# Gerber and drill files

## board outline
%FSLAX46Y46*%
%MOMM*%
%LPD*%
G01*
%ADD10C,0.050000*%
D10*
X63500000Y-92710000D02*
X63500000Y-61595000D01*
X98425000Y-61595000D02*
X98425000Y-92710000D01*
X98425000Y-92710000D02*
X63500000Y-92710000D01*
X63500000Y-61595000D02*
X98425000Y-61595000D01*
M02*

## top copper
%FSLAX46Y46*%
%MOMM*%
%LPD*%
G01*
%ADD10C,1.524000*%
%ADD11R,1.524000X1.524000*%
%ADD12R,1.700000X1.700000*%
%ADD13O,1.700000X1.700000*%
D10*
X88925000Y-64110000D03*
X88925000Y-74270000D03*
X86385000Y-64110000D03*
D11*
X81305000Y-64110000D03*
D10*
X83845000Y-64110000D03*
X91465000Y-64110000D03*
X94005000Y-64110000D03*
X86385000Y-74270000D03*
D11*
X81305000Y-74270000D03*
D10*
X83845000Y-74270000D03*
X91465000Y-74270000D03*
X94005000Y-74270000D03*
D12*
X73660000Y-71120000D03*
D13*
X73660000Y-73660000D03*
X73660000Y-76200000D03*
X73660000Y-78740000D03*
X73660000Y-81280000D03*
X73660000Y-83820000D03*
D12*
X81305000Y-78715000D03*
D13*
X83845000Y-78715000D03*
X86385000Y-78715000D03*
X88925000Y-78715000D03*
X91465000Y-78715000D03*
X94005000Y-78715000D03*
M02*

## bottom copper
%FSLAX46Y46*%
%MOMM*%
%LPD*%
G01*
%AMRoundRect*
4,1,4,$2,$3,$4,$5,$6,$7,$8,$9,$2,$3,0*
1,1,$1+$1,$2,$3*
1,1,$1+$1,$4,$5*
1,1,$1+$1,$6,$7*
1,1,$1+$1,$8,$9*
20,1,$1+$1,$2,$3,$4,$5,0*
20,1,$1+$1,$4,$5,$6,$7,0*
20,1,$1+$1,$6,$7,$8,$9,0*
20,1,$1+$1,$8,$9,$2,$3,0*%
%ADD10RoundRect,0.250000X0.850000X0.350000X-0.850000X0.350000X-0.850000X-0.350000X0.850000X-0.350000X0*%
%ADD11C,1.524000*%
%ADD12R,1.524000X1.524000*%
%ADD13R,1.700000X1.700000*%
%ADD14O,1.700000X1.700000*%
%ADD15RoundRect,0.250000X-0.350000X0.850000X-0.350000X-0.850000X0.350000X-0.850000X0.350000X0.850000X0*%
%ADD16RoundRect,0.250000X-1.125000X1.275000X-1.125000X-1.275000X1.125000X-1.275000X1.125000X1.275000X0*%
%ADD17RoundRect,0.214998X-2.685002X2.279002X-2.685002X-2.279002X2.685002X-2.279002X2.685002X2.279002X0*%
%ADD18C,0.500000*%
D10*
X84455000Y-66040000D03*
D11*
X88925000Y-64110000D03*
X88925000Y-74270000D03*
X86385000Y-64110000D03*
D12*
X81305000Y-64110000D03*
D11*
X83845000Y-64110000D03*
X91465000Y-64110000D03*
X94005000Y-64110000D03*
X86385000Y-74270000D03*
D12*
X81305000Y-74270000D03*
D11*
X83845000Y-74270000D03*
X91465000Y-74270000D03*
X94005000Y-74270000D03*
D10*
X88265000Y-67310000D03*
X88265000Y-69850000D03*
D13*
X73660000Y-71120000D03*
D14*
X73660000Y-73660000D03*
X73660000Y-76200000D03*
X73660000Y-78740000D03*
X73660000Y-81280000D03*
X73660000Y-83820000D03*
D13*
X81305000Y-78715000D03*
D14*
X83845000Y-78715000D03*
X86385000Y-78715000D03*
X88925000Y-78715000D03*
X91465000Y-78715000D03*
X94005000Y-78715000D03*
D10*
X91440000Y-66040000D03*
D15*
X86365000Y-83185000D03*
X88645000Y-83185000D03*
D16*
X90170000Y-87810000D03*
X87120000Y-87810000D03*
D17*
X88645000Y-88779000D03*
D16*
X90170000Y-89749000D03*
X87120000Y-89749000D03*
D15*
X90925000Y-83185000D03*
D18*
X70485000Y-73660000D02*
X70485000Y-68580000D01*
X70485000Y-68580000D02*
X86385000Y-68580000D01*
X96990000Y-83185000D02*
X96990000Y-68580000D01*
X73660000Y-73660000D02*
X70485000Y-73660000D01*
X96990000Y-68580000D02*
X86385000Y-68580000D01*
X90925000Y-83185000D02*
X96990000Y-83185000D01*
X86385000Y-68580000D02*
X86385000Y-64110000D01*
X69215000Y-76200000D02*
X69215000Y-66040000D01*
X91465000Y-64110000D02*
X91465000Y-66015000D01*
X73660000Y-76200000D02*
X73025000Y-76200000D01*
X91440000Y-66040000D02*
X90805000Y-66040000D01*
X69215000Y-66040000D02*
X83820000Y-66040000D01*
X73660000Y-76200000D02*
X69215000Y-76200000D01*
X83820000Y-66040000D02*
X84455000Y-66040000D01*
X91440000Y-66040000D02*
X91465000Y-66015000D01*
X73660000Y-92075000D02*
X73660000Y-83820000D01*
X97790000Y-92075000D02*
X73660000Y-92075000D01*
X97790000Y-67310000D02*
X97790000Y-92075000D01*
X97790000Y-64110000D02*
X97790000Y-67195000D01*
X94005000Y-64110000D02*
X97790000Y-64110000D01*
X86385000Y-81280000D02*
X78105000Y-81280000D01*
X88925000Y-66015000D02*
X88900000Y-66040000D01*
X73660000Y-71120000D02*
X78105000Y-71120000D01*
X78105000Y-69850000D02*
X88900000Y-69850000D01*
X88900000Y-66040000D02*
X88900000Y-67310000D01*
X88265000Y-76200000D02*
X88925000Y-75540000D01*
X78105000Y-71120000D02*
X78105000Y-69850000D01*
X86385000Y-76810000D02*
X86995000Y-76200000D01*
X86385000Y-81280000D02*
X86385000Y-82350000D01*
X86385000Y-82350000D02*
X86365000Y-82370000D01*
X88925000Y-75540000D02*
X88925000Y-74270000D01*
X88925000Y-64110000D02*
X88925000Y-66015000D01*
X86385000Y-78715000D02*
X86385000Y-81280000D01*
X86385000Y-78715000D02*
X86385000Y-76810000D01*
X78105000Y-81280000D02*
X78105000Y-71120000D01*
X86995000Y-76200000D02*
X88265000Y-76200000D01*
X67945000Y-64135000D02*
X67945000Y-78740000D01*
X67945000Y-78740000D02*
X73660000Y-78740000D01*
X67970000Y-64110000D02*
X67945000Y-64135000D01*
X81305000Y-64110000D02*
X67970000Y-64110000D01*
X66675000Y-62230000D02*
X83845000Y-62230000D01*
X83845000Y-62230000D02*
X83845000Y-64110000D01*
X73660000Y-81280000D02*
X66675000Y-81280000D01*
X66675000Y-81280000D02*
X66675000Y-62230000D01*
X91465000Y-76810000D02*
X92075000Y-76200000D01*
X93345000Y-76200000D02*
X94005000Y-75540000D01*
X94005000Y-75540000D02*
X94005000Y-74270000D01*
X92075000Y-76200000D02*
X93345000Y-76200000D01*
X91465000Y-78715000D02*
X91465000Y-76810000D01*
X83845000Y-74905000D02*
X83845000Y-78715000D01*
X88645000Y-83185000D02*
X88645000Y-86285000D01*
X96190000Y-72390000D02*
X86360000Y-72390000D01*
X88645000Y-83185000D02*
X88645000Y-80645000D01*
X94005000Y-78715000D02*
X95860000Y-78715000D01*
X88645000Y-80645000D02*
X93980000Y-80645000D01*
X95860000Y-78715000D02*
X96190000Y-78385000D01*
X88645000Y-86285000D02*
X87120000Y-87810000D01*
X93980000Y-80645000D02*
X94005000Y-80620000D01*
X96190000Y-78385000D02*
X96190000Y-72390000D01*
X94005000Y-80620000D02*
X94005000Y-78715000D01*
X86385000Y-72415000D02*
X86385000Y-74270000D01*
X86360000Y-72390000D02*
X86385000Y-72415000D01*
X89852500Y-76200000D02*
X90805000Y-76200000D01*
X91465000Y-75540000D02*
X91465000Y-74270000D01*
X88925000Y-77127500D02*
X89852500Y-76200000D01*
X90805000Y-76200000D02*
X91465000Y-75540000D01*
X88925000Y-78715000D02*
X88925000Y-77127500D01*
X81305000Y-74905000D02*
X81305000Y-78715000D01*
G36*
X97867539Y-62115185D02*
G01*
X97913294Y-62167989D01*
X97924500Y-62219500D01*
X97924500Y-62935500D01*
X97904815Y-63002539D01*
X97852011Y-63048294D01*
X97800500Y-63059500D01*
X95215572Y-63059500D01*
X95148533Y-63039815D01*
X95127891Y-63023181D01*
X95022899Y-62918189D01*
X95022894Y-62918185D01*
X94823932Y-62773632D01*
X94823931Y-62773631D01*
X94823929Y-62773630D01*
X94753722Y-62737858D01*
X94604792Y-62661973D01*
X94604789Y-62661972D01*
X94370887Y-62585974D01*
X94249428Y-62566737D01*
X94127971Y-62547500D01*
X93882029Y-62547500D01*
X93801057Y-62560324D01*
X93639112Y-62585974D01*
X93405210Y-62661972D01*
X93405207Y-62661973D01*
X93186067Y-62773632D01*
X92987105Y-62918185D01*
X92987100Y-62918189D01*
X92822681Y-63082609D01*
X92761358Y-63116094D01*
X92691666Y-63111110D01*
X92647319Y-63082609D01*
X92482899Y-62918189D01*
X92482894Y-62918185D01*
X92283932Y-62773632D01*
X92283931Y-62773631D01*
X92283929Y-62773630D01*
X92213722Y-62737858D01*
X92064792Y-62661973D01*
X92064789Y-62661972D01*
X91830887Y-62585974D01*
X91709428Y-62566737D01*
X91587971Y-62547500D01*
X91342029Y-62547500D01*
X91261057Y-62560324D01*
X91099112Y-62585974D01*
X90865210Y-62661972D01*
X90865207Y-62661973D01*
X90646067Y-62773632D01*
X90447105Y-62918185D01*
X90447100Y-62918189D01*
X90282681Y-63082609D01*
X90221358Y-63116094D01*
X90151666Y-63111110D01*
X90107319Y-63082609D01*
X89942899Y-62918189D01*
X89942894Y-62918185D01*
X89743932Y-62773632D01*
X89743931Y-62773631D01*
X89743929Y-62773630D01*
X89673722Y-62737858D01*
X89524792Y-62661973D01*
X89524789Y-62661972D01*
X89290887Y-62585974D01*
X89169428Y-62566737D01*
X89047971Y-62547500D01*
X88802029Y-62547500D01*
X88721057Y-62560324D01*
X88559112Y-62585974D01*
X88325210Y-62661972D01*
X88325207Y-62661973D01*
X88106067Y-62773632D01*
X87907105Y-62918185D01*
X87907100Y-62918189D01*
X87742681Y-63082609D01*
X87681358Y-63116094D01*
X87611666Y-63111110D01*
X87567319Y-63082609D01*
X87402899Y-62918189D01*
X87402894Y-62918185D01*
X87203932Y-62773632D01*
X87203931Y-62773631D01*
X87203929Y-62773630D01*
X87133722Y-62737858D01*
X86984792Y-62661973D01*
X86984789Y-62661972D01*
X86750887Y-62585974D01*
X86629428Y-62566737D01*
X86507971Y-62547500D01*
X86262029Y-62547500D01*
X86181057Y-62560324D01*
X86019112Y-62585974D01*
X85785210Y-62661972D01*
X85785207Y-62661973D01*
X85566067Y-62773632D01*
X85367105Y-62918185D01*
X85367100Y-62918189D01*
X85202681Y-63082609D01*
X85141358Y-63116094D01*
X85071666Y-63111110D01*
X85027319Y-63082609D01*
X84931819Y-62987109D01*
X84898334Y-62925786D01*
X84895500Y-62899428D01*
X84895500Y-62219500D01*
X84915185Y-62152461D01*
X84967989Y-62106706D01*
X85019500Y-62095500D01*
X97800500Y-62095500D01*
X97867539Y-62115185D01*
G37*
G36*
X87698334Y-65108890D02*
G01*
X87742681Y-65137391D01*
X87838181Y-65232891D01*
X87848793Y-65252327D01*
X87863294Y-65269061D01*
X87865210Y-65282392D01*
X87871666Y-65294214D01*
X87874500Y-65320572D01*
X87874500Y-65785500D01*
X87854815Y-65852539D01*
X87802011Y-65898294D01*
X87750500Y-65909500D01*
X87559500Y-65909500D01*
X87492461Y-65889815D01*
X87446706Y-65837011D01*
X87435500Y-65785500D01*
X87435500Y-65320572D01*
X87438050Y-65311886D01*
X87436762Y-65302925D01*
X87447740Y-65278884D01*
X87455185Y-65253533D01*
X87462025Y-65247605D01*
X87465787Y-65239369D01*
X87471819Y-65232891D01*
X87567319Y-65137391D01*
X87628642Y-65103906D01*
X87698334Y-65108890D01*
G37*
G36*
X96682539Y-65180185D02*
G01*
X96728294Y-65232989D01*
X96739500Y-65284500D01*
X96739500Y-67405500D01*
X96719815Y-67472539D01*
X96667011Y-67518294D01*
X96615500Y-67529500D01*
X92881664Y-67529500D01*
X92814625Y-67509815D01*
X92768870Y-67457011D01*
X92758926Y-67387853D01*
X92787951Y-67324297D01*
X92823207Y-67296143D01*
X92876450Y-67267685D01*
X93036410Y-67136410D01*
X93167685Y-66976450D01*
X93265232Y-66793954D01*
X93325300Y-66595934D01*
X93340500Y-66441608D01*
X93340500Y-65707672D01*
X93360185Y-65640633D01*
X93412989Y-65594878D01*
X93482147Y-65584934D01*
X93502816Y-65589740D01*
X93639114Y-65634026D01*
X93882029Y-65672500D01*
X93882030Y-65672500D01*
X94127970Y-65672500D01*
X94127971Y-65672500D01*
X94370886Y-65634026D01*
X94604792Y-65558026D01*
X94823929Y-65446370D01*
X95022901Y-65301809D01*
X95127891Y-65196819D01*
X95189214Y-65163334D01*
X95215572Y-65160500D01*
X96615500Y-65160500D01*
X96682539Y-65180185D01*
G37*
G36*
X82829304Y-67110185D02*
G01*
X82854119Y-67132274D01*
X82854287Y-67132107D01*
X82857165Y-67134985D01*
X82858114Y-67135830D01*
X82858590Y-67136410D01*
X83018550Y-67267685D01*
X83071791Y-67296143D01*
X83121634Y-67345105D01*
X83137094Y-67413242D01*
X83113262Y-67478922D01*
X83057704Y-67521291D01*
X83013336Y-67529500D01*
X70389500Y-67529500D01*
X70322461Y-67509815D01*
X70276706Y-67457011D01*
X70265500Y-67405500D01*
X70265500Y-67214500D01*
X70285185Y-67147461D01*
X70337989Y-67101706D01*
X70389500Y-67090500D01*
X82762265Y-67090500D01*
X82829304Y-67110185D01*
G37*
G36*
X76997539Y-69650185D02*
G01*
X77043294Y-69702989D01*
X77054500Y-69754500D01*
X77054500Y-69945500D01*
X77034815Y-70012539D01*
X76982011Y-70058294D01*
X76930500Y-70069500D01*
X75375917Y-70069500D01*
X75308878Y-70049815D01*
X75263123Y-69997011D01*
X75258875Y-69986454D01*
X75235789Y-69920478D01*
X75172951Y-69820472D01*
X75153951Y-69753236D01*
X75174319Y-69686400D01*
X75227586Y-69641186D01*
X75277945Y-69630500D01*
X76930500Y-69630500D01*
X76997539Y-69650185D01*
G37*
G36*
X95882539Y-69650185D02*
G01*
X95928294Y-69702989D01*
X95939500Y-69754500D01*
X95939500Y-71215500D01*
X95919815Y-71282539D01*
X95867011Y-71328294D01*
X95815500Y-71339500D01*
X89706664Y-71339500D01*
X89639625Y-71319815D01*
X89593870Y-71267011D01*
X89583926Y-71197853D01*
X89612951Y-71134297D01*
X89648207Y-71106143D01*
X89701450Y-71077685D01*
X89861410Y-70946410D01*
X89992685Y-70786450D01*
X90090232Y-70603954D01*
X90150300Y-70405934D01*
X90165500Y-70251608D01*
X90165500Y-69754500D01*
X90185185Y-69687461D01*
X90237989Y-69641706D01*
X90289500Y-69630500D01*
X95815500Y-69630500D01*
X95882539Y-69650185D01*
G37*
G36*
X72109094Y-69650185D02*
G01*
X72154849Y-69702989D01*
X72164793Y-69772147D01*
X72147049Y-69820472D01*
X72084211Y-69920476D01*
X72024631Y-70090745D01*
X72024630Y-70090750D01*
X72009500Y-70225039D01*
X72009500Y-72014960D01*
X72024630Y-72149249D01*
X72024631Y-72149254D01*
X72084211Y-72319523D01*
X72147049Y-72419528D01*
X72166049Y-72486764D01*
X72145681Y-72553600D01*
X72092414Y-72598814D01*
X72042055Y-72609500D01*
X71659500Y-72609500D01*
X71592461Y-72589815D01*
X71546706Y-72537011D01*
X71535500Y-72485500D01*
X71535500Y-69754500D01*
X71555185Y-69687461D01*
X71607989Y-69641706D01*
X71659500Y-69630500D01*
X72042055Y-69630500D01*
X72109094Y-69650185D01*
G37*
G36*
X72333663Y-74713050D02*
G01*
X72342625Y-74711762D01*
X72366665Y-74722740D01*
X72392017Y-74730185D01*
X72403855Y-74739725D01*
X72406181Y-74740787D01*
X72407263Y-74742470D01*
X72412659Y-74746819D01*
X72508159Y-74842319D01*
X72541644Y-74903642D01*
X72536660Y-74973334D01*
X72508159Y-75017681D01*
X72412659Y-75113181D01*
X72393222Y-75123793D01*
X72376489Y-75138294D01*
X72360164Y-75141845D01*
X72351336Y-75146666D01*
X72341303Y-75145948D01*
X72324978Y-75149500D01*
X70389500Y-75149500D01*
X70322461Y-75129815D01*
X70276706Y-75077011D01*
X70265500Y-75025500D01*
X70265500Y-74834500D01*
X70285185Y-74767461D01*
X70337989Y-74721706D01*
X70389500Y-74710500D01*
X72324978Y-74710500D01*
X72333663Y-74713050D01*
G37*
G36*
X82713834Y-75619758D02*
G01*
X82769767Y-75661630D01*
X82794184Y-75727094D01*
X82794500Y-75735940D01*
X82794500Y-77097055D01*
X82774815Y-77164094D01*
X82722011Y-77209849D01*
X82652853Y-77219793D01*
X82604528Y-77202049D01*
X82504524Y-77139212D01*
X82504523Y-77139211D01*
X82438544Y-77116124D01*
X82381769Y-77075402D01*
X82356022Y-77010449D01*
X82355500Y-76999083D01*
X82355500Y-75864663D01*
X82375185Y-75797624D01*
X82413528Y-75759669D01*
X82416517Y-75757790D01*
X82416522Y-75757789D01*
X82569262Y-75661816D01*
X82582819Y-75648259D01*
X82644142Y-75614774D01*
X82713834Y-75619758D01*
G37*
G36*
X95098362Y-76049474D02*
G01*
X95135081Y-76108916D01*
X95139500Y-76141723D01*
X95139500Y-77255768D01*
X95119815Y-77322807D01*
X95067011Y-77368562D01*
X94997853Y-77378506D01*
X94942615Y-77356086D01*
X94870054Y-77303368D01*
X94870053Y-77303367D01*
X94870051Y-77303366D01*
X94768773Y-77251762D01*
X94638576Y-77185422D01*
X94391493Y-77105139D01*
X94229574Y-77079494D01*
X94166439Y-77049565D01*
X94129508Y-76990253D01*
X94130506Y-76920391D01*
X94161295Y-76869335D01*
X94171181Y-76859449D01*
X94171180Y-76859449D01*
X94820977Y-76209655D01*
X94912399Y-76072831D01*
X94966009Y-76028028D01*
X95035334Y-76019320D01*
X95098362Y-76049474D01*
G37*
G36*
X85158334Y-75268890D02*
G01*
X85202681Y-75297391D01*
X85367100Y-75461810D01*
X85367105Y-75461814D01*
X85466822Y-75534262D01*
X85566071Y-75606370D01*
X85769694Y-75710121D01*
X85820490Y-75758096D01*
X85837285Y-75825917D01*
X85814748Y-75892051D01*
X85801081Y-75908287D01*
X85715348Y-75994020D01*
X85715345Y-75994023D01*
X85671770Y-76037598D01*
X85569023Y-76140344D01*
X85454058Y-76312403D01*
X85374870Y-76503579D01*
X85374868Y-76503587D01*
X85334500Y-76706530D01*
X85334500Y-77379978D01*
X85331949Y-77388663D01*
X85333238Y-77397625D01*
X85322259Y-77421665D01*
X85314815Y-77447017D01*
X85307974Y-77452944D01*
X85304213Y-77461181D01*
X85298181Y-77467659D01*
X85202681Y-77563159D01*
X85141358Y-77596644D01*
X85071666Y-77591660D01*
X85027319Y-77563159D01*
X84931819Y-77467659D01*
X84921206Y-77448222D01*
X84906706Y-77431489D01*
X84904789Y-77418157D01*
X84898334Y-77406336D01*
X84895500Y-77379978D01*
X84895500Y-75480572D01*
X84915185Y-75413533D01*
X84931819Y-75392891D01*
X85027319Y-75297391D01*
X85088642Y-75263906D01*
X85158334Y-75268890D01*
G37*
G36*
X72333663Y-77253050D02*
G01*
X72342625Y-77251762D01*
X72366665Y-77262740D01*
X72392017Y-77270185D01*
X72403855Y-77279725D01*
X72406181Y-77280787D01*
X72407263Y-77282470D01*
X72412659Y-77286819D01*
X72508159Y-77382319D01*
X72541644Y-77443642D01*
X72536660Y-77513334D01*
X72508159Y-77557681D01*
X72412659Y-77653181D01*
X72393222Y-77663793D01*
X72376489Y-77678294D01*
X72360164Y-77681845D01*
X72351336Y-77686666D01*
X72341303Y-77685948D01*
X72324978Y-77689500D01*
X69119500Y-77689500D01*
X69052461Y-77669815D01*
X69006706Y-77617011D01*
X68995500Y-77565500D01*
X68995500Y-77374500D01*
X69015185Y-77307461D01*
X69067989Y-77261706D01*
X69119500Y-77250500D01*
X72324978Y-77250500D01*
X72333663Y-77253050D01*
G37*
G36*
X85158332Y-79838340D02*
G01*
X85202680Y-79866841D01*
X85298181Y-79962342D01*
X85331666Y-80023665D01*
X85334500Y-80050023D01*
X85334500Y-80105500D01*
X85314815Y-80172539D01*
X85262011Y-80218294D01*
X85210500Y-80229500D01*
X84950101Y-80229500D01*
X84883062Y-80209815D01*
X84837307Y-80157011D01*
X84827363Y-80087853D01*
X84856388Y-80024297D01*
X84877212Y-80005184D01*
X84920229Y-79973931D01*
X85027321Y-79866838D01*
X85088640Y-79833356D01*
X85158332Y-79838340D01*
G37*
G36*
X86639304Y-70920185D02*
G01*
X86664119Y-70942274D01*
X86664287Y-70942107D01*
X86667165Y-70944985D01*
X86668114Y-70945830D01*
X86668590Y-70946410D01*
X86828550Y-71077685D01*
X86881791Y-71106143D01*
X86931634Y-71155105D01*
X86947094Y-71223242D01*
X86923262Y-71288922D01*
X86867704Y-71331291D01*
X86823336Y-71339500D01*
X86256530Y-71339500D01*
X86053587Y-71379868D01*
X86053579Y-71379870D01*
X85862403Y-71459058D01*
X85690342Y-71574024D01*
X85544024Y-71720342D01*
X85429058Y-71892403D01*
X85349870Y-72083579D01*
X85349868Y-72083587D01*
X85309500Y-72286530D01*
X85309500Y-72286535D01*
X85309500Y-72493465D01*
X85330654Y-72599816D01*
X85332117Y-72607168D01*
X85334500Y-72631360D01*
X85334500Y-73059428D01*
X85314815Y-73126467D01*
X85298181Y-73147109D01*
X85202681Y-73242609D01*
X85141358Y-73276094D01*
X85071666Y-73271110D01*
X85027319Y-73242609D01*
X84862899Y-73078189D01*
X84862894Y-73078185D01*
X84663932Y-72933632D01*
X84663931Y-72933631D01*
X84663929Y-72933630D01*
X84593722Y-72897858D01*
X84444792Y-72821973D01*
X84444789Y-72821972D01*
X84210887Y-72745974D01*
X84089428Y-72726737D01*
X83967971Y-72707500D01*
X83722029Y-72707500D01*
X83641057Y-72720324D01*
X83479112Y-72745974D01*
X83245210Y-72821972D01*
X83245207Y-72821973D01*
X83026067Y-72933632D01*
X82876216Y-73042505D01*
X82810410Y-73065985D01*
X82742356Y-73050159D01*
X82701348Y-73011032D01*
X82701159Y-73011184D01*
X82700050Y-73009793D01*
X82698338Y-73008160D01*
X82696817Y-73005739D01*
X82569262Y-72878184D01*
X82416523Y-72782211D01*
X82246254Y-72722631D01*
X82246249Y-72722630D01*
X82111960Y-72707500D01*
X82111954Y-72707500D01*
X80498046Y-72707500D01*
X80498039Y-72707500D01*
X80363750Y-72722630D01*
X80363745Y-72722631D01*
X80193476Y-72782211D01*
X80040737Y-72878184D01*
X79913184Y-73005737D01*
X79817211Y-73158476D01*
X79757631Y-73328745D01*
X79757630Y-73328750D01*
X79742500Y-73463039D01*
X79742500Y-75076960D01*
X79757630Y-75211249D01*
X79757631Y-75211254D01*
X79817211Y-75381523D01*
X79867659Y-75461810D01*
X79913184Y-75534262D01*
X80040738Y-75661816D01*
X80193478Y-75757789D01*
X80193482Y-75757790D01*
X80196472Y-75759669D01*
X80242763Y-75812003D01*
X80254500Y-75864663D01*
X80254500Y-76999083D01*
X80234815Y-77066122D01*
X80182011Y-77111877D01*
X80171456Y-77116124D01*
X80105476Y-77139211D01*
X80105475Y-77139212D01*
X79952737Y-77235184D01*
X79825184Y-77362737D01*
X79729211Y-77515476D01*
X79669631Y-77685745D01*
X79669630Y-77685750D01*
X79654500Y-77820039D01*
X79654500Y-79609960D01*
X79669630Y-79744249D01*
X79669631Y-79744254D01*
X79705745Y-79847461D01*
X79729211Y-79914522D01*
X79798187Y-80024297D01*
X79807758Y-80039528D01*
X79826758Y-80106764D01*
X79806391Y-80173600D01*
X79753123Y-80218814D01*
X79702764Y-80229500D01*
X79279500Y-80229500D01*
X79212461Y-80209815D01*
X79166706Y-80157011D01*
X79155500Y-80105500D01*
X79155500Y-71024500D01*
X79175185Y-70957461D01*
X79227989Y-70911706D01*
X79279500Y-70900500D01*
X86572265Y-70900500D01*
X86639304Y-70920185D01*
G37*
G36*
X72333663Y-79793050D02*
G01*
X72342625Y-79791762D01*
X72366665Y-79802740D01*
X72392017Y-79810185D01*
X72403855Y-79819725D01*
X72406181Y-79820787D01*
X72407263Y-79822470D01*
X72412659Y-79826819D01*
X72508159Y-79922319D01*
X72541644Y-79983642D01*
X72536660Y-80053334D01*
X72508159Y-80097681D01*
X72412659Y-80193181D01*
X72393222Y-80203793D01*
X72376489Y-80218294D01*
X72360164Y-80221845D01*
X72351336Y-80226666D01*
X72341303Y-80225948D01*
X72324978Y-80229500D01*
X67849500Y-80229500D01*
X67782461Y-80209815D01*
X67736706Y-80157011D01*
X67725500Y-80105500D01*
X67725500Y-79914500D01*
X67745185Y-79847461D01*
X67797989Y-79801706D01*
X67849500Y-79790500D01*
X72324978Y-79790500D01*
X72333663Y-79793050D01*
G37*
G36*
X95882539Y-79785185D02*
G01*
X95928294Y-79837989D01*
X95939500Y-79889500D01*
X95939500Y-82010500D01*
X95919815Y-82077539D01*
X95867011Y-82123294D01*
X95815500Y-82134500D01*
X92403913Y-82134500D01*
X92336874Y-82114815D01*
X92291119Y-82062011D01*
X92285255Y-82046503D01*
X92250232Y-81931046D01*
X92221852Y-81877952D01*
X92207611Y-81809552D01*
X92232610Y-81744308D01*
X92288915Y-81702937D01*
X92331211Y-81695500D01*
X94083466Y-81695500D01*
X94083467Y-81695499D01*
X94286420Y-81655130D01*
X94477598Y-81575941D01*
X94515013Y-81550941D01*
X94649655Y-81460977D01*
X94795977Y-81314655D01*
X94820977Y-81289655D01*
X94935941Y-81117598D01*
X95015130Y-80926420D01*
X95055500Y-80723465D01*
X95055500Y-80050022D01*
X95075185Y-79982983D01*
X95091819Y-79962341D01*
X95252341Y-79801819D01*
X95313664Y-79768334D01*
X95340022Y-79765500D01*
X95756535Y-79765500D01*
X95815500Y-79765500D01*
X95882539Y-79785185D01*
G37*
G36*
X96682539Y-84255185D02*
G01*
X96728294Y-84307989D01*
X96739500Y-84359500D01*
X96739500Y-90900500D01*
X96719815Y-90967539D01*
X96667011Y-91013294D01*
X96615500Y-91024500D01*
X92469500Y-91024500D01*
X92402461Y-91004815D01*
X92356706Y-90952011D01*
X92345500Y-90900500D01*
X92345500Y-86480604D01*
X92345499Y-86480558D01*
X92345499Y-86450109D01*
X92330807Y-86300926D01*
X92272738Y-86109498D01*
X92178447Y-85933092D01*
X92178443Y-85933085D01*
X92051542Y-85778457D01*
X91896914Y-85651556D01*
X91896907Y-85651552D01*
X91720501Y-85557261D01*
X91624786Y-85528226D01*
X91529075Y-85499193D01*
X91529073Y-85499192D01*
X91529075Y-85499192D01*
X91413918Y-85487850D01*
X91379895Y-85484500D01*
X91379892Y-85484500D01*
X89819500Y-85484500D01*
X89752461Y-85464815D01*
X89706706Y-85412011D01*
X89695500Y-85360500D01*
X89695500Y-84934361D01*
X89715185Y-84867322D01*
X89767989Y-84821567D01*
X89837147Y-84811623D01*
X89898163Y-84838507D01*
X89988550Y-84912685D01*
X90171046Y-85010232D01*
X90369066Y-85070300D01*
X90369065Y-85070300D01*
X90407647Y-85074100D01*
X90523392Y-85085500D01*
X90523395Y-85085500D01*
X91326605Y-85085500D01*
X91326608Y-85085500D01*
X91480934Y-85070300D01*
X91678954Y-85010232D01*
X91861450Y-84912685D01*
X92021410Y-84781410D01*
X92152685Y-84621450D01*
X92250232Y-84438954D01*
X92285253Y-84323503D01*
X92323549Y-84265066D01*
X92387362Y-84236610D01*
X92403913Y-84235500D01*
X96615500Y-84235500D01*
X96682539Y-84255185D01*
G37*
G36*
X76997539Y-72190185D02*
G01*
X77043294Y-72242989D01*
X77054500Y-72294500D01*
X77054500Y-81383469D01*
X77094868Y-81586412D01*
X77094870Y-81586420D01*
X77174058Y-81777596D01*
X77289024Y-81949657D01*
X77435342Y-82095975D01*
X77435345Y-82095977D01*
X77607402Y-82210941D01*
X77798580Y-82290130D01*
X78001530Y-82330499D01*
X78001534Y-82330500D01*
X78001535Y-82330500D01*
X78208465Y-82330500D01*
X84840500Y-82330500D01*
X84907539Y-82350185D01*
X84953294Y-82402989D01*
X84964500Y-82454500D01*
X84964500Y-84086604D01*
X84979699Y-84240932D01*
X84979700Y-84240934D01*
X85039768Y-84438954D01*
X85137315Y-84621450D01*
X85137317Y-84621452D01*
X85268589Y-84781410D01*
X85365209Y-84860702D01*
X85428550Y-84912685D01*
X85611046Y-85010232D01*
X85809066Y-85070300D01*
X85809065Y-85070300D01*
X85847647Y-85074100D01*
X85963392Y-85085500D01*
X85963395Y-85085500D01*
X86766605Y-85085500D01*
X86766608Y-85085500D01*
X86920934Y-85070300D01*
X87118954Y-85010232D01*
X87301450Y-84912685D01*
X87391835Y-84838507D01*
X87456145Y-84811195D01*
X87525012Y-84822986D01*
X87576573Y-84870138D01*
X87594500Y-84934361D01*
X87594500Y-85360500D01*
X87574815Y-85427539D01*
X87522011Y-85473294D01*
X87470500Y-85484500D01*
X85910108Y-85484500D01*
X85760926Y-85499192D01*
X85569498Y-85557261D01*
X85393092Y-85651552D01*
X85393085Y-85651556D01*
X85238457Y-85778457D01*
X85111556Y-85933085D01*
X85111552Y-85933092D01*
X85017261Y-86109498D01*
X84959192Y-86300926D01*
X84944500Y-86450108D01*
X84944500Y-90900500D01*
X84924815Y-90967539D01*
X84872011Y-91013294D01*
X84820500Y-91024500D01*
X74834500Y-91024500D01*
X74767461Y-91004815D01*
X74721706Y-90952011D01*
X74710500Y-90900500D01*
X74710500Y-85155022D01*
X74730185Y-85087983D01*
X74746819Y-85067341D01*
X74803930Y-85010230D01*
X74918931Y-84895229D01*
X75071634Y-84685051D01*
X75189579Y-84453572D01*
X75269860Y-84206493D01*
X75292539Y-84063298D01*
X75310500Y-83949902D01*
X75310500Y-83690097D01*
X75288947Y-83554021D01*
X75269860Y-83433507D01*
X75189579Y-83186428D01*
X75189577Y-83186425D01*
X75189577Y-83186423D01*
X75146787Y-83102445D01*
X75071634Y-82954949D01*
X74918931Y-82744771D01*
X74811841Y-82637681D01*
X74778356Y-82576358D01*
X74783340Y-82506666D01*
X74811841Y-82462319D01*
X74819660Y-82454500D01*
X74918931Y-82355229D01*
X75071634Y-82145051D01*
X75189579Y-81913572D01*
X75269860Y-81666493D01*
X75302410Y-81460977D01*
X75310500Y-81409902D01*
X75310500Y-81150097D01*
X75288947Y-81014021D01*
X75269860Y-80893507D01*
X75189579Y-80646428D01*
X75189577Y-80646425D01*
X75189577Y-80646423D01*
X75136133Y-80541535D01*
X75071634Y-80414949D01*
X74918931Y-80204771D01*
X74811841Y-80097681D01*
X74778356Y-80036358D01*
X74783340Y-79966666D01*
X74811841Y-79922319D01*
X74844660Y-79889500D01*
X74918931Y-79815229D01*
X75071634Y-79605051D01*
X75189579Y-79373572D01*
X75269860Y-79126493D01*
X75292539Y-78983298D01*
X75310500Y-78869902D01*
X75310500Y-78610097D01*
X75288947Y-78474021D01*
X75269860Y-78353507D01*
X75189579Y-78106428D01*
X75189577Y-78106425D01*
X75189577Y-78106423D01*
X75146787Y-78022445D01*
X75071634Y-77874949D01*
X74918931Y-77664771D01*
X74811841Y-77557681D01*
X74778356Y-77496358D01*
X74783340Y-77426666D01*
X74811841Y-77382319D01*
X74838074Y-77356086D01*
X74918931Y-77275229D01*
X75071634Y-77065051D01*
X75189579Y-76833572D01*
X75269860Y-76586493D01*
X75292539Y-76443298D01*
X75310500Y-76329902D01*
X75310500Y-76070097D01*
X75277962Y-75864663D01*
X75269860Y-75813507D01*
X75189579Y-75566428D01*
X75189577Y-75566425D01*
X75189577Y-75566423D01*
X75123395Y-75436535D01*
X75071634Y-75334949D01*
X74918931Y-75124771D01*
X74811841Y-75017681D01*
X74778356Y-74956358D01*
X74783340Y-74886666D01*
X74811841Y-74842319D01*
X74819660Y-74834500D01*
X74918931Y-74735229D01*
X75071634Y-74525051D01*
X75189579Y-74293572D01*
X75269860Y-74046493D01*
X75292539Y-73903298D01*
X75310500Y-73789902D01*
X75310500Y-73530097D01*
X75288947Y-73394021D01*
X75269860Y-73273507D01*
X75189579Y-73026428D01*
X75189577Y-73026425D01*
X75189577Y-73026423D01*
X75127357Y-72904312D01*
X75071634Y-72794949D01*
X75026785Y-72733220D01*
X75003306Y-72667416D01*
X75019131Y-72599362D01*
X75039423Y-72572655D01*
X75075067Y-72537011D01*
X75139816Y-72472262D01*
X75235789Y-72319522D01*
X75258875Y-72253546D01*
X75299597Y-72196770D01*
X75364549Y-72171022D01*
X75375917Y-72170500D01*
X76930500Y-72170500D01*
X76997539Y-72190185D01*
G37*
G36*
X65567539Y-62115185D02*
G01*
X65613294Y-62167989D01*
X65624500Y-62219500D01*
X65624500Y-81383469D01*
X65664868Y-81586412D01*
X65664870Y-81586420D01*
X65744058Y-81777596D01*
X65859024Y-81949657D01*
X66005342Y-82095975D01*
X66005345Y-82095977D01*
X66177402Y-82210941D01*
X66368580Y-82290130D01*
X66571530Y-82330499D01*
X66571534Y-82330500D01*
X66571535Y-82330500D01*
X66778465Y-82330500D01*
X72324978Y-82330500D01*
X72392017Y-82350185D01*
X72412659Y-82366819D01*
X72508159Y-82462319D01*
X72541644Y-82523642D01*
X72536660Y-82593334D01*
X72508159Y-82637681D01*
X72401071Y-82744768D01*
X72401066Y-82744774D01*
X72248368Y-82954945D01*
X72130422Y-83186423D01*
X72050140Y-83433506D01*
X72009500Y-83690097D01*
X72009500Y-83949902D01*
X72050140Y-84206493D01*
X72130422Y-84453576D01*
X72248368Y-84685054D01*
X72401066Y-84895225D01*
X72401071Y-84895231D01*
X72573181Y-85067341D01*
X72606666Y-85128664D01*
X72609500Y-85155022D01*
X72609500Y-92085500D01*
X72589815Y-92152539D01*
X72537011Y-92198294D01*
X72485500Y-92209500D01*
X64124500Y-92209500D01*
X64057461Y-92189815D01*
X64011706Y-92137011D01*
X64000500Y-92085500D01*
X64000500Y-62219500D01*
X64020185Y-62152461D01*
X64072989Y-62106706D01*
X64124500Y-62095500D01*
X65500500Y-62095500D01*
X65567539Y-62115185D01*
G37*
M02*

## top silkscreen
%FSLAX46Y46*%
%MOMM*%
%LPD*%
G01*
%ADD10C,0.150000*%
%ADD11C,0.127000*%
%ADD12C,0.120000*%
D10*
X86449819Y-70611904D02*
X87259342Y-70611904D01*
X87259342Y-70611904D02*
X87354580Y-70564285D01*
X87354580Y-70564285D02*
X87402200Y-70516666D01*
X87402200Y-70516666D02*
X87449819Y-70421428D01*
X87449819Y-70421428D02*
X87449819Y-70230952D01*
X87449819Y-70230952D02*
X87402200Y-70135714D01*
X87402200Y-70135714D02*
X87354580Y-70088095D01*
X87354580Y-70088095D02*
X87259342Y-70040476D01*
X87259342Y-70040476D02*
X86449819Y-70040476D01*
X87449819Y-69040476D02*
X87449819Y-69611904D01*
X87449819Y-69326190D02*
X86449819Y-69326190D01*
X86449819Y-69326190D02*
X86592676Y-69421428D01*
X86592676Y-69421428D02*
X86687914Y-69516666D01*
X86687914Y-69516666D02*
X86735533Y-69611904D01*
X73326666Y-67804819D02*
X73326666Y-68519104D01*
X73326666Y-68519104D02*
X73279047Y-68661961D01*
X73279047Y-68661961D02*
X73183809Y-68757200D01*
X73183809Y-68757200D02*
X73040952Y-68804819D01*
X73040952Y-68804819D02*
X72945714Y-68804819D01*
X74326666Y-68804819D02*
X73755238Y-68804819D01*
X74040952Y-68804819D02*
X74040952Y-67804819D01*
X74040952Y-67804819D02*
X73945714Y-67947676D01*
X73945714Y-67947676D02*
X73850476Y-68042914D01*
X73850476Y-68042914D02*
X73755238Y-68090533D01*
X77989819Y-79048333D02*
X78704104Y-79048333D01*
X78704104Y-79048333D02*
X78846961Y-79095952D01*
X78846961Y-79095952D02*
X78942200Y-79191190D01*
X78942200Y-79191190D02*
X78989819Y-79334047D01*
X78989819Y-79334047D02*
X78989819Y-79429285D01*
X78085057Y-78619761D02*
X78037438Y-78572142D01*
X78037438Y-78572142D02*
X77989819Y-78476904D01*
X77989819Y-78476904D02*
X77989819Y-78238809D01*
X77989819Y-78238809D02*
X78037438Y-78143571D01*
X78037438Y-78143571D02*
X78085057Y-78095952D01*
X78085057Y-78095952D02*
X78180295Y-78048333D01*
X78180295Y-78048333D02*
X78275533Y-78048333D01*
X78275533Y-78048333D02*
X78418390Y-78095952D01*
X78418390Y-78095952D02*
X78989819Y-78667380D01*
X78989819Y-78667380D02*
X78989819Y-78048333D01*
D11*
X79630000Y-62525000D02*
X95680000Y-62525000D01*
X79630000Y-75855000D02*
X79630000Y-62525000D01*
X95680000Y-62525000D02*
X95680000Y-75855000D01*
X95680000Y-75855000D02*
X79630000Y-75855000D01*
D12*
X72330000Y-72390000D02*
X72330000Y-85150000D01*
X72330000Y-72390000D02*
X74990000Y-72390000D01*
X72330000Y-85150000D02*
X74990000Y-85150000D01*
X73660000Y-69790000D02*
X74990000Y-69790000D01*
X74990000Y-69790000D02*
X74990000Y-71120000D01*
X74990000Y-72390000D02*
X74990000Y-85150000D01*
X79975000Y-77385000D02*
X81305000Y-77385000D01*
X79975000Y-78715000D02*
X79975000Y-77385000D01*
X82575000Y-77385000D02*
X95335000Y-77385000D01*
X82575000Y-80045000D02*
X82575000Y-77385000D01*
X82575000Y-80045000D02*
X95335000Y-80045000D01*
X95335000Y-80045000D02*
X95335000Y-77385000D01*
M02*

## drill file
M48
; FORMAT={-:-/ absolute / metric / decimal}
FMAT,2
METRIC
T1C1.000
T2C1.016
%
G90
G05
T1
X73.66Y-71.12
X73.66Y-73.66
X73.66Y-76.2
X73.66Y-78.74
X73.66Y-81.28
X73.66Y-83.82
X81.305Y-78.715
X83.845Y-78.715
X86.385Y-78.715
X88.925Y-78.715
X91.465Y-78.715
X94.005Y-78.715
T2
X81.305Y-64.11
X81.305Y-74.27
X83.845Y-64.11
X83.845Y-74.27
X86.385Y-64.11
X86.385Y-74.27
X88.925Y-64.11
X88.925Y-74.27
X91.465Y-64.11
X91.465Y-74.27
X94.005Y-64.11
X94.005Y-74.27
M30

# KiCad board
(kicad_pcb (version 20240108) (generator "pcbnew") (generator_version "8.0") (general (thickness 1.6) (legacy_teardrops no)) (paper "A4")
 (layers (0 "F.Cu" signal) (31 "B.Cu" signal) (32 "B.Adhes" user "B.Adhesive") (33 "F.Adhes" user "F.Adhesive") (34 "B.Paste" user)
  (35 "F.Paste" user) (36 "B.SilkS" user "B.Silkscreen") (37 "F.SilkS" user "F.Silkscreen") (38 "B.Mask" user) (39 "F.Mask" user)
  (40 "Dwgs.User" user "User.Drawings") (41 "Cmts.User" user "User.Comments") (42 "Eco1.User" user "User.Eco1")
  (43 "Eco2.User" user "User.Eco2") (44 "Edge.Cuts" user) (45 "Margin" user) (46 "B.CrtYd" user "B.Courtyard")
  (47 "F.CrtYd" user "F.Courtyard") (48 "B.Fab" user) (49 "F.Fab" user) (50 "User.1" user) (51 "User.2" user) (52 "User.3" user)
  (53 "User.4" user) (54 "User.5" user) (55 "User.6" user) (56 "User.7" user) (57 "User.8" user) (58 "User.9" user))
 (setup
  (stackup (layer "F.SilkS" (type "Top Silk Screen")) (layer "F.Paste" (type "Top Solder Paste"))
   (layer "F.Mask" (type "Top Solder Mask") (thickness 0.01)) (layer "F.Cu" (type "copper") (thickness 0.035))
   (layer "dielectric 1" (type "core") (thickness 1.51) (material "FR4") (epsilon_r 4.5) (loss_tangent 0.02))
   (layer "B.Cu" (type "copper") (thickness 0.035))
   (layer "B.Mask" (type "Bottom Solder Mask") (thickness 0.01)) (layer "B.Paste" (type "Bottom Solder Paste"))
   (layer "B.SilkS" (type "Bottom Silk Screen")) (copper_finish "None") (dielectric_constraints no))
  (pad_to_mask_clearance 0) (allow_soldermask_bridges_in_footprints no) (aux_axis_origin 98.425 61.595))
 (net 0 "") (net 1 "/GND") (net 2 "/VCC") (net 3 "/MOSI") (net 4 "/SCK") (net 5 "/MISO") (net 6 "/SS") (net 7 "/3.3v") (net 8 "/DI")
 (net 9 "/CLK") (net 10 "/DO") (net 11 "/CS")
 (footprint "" (layer "F.Cu") (at 84.455 66.04 -90)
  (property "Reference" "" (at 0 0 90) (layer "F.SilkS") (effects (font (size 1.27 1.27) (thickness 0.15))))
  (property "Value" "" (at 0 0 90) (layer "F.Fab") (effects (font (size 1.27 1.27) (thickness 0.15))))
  (pad "1" smd roundrect (at 0 0 180) (size 2.2 1.2) (layers "B.Cu" "B.Paste" "B.Mask") (roundrect_rratio 0.208333)))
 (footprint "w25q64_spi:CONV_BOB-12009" (layer "F.Cu") (at 87.655 69.19 90)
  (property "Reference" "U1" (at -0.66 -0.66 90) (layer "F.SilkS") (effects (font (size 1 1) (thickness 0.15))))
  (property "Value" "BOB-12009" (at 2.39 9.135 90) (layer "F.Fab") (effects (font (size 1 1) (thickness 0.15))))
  (fp_line (start 6.665 -8.025) (end 6.665 8.025) (stroke (width 0.127) (type solid)) (layer "F.SilkS"))
  (fp_line (start -6.665 -8.025) (end 6.665 -8.025) (stroke (width 0.127) (type solid)) (layer "F.SilkS"))
  (fp_line (start 6.665 8.025) (end -6.665 8.025) (stroke (width 0.127) (type solid)) (layer "F.SilkS"))
  (fp_line (start -6.665 8.025) (end -6.665 -8.025) (stroke (width 0.127) (type solid)) (layer "F.SilkS"))
  (pad "GND_1" thru_hole circle (at 5.08 1.27 90) (size 1.524 1.524) (drill 1.016) (layers "*.Cu" "*.Mask") (remove_unused_layers no)
   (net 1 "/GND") (solder_mask_margin 0.102))
  (pad "GND_2" thru_hole circle (at -5.08 1.27 90) (size 1.524 1.524) (drill 1.016) (layers "*.Cu" "*.Mask") (remove_unused_layers no)
   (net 1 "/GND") (solder_mask_margin 0.102))
  (pad "HV" thru_hole circle (at 5.08 -1.27 90) (size 1.524 1.524) (drill 1.016) (layers "*.Cu" "*.Mask") (remove_unused_layers no)
   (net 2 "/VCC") (solder_mask_margin 0.102))
  (pad "HV1" thru_hole rect (at 5.08 -6.35 90) (size 1.524 1.524) (drill 1.016) (layers "*.Cu" "*.Mask") (remove_unused_layers no)
   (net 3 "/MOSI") (solder_mask_margin 0.102))
  (pad "HV2" thru_hole circle (at 5.08 -3.81 90) (size 1.524 1.524) (drill 1.016) (layers "*.Cu" "*.Mask") (remove_unused_layers no)
   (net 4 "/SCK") (solder_mask_margin 0.102))
  (pad "HV3" thru_hole circle (at 5.08 3.81 90) (size 1.524 1.524) (drill 1.016) (layers "*.Cu" "*.Mask") (remove_unused_layers no)
   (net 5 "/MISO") (solder_mask_margin 0.102))
  (pad "HV4" thru_hole circle (at 5.08 6.35 90) (size 1.524 1.524) (drill 1.016) (layers "*.Cu" "*.Mask") (remove_unused_layers no)
   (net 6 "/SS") (solder_mask_margin 0.102))
  (pad "LV" thru_hole circle (at -5.08 -1.27 90) (size 1.524 1.524) (drill 1.016) (layers "*.Cu" "*.Mask") (remove_unused_layers no)
   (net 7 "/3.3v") (solder_mask_margin 0.102))
  (pad "LV1" thru_hole rect (at -5.08 -6.35 90) (size 1.524 1.524) (drill 1.016) (layers "*.Cu" "*.Mask") (remove_unused_layers no)
   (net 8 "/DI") (solder_mask_margin 0.102))
  (pad "LV2" thru_hole circle (at -5.08 -3.81 90) (size 1.524 1.524) (drill 1.016) (layers "*.Cu" "*.Mask") (remove_unused_layers no)
   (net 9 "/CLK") (solder_mask_margin 0.102))
  (pad "LV3" thru_hole circle (at -5.08 3.81 90) (size 1.524 1.524) (drill 1.016) (layers "*.Cu" "*.Mask") (remove_unused_layers no)
   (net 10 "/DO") (solder_mask_margin 0.102))
  (pad "LV4" thru_hole circle (at -5.08 6.35 90) (size 1.524 1.524) (drill 1.016) (layers "*.Cu" "*.Mask") (remove_unused_layers no)
   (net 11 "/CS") (solder_mask_margin 0.102)))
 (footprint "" (layer "F.Cu") (at 88.265 67.31 -90)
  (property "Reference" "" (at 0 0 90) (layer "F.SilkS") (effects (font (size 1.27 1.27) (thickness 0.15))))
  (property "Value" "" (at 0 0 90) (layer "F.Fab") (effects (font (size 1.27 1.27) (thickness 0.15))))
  (pad "1" smd roundrect (at 0 0 180) (size 2.2 1.2) (layers "B.Cu" "B.Paste" "B.Mask") (roundrect_rratio 0.208333)))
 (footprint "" (layer "F.Cu") (at 88.265 69.85 -90)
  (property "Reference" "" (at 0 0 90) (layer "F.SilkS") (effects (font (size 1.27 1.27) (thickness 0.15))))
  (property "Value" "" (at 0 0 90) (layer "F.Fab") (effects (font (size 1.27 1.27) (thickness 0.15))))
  (pad "1" smd roundrect (at 0 0 180) (size 2.2 1.2) (layers "B.Cu" "B.Paste" "B.Mask") (roundrect_rratio 0.208333)))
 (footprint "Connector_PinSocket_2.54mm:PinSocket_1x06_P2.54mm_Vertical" (layer "F.Cu") (at 73.66 71.12)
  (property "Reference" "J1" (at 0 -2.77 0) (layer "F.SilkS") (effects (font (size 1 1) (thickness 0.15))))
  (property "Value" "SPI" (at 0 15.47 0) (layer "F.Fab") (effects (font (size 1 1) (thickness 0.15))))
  (fp_line (start -1.33 1.27) (end -1.33 14.03) (stroke (width 0.12) (type solid)) (layer "F.SilkS"))
  (fp_line (start -1.33 1.27) (end 1.33 1.27) (stroke (width 0.12) (type solid)) (layer "F.SilkS"))
  (fp_line (start -1.33 14.03) (end 1.33 14.03) (stroke (width 0.12) (type solid)) (layer "F.SilkS"))
  (fp_line (start 0 -1.33) (end 1.33 -1.33) (stroke (width 0.12) (type solid)) (layer "F.SilkS"))
  (fp_line (start 1.33 -1.33) (end 1.33 0) (stroke (width 0.12) (type solid)) (layer "F.SilkS"))
  (fp_line (start 1.33 1.27) (end 1.33 14.03) (stroke (width 0.12) (type solid)) (layer "F.SilkS"))
  (pad "1" thru_hole rect (at 0 0) (size 1.7 1.7) (drill 1) (layers "*.Cu" "*.Mask") (remove_unused_layers no) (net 1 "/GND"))
  (pad "2" thru_hole oval (at 0 2.54) (size 1.7 1.7) (drill 1) (layers "*.Cu" "*.Mask") (remove_unused_layers no) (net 2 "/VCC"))
  (pad "3" thru_hole oval (at 0 5.08) (size 1.7 1.7) (drill 1) (layers "*.Cu" "*.Mask") (remove_unused_layers no) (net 5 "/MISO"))
  (pad "4" thru_hole oval (at 0 7.62) (size 1.7 1.7) (drill 1) (layers "*.Cu" "*.Mask") (remove_unused_layers no) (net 3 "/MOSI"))
  (pad "5" thru_hole oval (at 0 10.16) (size 1.7 1.7) (drill 1) (layers "*.Cu" "*.Mask") (remove_unused_layers no) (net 4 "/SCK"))
  (pad "6" thru_hole oval (at 0 12.7) (size 1.7 1.7) (drill 1) (layers "*.Cu" "*.Mask") (remove_unused_layers no) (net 6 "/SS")))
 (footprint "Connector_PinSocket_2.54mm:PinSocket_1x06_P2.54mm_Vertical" (layer "F.Cu") (at 81.305 78.715 90)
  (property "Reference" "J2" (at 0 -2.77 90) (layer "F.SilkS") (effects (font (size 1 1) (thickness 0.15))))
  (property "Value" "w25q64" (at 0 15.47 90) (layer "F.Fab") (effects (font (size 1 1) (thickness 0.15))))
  (fp_line (start 1.33 -1.33) (end 1.33 0) (stroke (width 0.12) (type solid)) (layer "F.SilkS"))
  (fp_line (start 0 -1.33) (end 1.33 -1.33) (stroke (width 0.12) (type solid)) (layer "F.SilkS"))
  (fp_line (start 1.33 1.27) (end 1.33 14.03) (stroke (width 0.12) (type solid)) (layer "F.SilkS"))
  (fp_line (start -1.33 1.27) (end 1.33 1.27) (stroke (width 0.12) (type solid)) (layer "F.SilkS"))
  (fp_line (start -1.33 1.27) (end -1.33 14.03) (stroke (width 0.12) (type solid)) (layer "F.SilkS"))
  (fp_line (start -1.33 14.03) (end 1.33 14.03) (stroke (width 0.12) (type solid)) (layer "F.SilkS"))
  (pad "1" thru_hole rect (at 0 0 90) (size 1.7 1.7) (drill 1) (layers "*.Cu" "*.Mask") (remove_unused_layers no) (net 8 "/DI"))
  (pad "2" thru_hole oval (at 0 2.54 90) (size 1.7 1.7) (drill 1) (layers "*.Cu" "*.Mask") (remove_unused_layers no) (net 9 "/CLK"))
  (pad "3" thru_hole oval (at 0 5.08 90) (size 1.7 1.7) (drill 1) (layers "*.Cu" "*.Mask") (remove_unused_layers no) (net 1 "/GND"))
  (pad "4" thru_hole oval (at 0 7.62 90) (size 1.7 1.7) (drill 1) (layers "*.Cu" "*.Mask") (remove_unused_layers no) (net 10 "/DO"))
  (pad "5" thru_hole oval (at 0 10.16 90) (size 1.7 1.7) (drill 1) (layers "*.Cu" "*.Mask") (remove_unused_layers no) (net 11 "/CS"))
  (pad "6" thru_hole oval (at 0 12.7 90) (size 1.7 1.7) (drill 1) (layers "*.Cu" "*.Mask") (remove_unused_layers no) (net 7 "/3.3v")))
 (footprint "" (layer "F.Cu") (at 91.44 66.04 -90)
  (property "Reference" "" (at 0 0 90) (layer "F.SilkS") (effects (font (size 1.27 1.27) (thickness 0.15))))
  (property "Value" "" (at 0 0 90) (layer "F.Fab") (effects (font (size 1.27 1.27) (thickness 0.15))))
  (pad "1" smd roundrect (at 0 0 180) (size 2.2 1.2) (layers "B.Cu" "B.Paste" "B.Mask") (roundrect_rratio 0.208333) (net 1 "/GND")))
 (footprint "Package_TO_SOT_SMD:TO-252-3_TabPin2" (layer "B.Cu") (at 88.645 88.225 -90)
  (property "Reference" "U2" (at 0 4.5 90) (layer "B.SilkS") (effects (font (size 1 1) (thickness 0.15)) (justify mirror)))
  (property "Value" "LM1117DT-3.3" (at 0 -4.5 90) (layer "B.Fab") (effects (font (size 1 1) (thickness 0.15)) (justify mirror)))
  (pad "1" smd roundrect (at -5.04 2.28 270) (size 2.2 1.2) (layers "B.Cu" "B.Paste" "B.Mask") (roundrect_rratio 0.208333) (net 1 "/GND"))
  (pad "2" smd roundrect (at -5.04 0 270) (size 2.2 1.2) (layers "B.Cu" "B.Paste" "B.Mask") (roundrect_rratio 0.208333) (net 7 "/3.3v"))
  (pad "2" smd roundrect (at -0.415 -1.525 270) (size 3.05 2.75) (layers "B.Cu" "B.Paste") (roundrect_rratio 0.090909) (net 7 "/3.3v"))
  (pad "2" smd roundrect (at -0.415 1.525 270) (size 3.05 2.75) (layers "B.Cu" "B.Paste") (roundrect_rratio 0.090909) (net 7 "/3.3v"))
  (pad "2" smd roundrect (at 0.554 0 270) (size 4.988 5.8) (layers "B.Cu" "B.Mask") (roundrect_rratio 0.043103) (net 7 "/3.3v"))
  (pad "2" smd roundrect (at 1.524 -1.525 270) (size 3.05 2.75) (layers "B.Cu" "B.Paste") (roundrect_rratio 0.090909) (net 7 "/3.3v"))
  (pad "2" smd roundrect (at 1.524 1.525 270) (size 3.05 2.75) (layers "B.Cu" "B.Paste") (roundrect_rratio 0.090909) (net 7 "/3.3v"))
  (pad "3" smd roundrect (at -5.04 -2.28 270) (size 2.2 1.2) (layers "B.Cu" "B.Paste" "B.Mask") (roundrect_rratio 0.208333) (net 2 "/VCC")))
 (gr_line (start 63.5 92.71) (end 63.5 61.595) (stroke (width 0.05) (type default)) (layer "Edge.Cuts"))
 (gr_line (start 98.425 61.595) (end 98.425 92.71) (stroke (width 0.05) (type default)) (layer "Edge.Cuts"))
 (gr_line (start 98.425 92.71) (end 63.5 92.71) (stroke (width 0.05) (type default)) (layer "Edge.Cuts"))
 (gr_line (start 63.5 61.595) (end 98.425 61.595) (stroke (width 0.05) (type default)) (layer "Edge.Cuts"))
 (segment (start 70.485 73.66) (end 70.485 68.58) (width 0.5) (layer "B.Cu") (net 2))
 (segment (start 70.485 68.58) (end 86.385 68.58) (width 0.5) (layer "B.Cu") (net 2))
 (segment (start 96.99 83.185) (end 96.99 68.58) (width 0.5) (layer "B.Cu") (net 2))
 (segment (start 73.66 73.66) (end 70.485 73.66) (width 0.5) (layer "B.Cu") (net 2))
 (segment (start 96.99 68.58) (end 86.385 68.58) (width 0.5) (layer "B.Cu") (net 2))
 (segment (start 90.925 83.185) (end 96.99 83.185) (width 0.5) (layer "B.Cu") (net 2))
 (segment (start 86.385 68.58) (end 86.385 64.11) (width 0.5) (layer "B.Cu") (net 2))
 (segment (start 69.215 76.2) (end 69.215 66.04) (width 0.5) (layer "B.Cu") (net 5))
 (segment (start 91.465 64.11) (end 91.465 66.015) (width 0.5) (layer "B.Cu") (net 5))
 (segment (start 73.66 76.2) (end 73.025 76.2) (width 0.5) (layer "B.Cu") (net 5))
 (segment (start 91.44 66.04) (end 90.805 66.04) (width 0.5) (layer "B.Cu") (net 5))
 (segment (start 69.215 66.04) (end 83.82 66.04) (width 0.5) (layer "B.Cu") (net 5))
 (segment (start 73.66 76.2) (end 69.215 76.2) (width 0.5) (layer "B.Cu") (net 5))
 (segment (start 83.82 66.04) (end 84.455 66.04) (width 0.5) (layer "B.Cu") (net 5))
 (segment (start 91.44 66.04) (end 91.465 66.015) (width 0.5) (layer "B.Cu") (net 5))
 (segment (start 73.66 92.075) (end 73.66 83.82) (width 0.5) (layer "B.Cu") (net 6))
 (segment (start 97.79 92.075) (end 73.66 92.075) (width 0.5) (layer "B.Cu") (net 6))
 (segment (start 97.79 67.31) (end 97.79 92.075) (width 0.5) (layer "B.Cu") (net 6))
 (segment (start 97.79 64.11) (end 97.79 67.195) (width 0.5) (layer "B.Cu") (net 6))
 (segment (start 94.005 64.11) (end 97.79 64.11) (width 0.5) (layer "B.Cu") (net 6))
 (segment (start 86.385 81.28) (end 78.105 81.28) (width 0.5) (layer "B.Cu") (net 1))
 (segment (start 88.925 66.015) (end 88.9 66.04) (width 0.5) (layer "B.Cu") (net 1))
 (segment (start 73.66 71.12) (end 78.105 71.12) (width 0.5) (layer "B.Cu") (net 1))
 (segment (start 78.105 69.85) (end 88.9 69.85) (width 0.5) (layer "B.Cu") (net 1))
 (segment (start 88.9 66.04) (end 88.9 67.31) (width 0.5) (layer "B.Cu") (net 1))
 (segment (start 88.265 76.2) (end 88.925 75.54) (width 0.5) (layer "B.Cu") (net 1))
 (segment (start 78.105 71.12) (end 78.105 69.85) (width 0.5) (layer "B.Cu") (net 1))
 (segment (start 86.385 76.81) (end 86.995 76.2) (width 0.5) (layer "B.Cu") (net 1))
 (segment (start 86.385 81.28) (end 86.385 82.35) (width 0.5) (layer "B.Cu") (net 1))
 (segment (start 86.385 82.35) (end 86.365 82.37) (width 0.5) (layer "B.Cu") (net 1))
 (segment (start 88.925 75.54) (end 88.925 74.27) (width 0.5) (layer "B.Cu") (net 1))
 (segment (start 88.925 64.11) (end 88.925 66.015) (width 0.5) (layer "B.Cu") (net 1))
 (segment (start 86.385 78.715) (end 86.385 81.28) (width 0.5) (layer "B.Cu") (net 1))
 (segment (start 86.385 78.715) (end 86.385 76.81) (width 0.5) (layer "B.Cu") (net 1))
 (segment (start 78.105 81.28) (end 78.105 71.12) (width 0.5) (layer "B.Cu") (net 1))
 (segment (start 86.995 76.2) (end 88.265 76.2) (width 0.5) (layer "B.Cu") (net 1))
 (segment (start 67.945 64.135) (end 67.945 78.74) (width 0.5) (layer "B.Cu") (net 3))
 (segment (start 67.945 78.74) (end 73.66 78.74) (width 0.5) (layer "B.Cu") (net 3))
 (segment (start 67.97 64.11) (end 67.945 64.135) (width 0.5) (layer "B.Cu") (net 3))
 (segment (start 81.305 64.11) (end 67.97 64.11) (width 0.5) (layer "B.Cu") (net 3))
 (segment (start 66.675 62.23) (end 83.845 62.23) (width 0.5) (layer "B.Cu") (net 4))
 (segment (start 83.845 62.23) (end 83.845 64.11) (width 0.5) (layer "B.Cu") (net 4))
 (segment (start 73.66 81.28) (end 66.675 81.28) (width 0.5) (layer "B.Cu") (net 4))
 (segment (start 66.675 81.28) (end 66.675 62.23) (width 0.5) (layer "B.Cu") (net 4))
 (segment (start 91.465 76.81) (end 92.075 76.2) (width 0.5) (layer "B.Cu") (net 11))
 (segment (start 93.345 76.2) (end 94.005 75.54) (width 0.5) (layer "B.Cu") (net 11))
 (segment (start 94.005 75.54) (end 94.005 74.27) (width 0.5) (layer "B.Cu") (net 11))
 (segment (start 92.075 76.2) (end 93.345 76.2) (width 0.5) (layer "B.Cu") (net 11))
 (segment (start 91.465 78.715) (end 91.465 76.81) (width 0.5) (layer "B.Cu") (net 11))
 (segment (start 83.845 74.905) (end 83.845 78.715) (width 0.5) (layer "B.Cu") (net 9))
 (segment (start 88.645 83.185) (end 88.645 86.285) (width 0.5) (layer "B.Cu") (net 7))
 (segment (start 96.19 72.39) (end 86.36 72.39) (width 0.5) (layer "B.Cu") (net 7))
 (segment (start 88.645 83.185) (end 88.645 80.645) (width 0.5) (layer "B.Cu") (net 7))
 (segment (start 94.005 78.715) (end 95.86 78.715) (width 0.5) (layer "B.Cu") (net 7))
 (segment (start 88.645 80.645) (end 93.98 80.645) (width 0.5) (layer "B.Cu") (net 7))
 (segment (start 95.86 78.715) (end 96.19 78.385) (width 0.5) (layer "B.Cu") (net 7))
 (segment (start 88.645 86.285) (end 87.12 87.81) (width 0.5) (layer "B.Cu") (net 7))
 (segment (start 93.98 80.645) (end 94.005 80.62) (width 0.5) (layer "B.Cu") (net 7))
 (segment (start 96.19 78.385) (end 96.19 72.39) (width 0.5) (layer "B.Cu") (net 7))
 (segment (start 94.005 80.62) (end 94.005 78.715) (width 0.5) (layer "B.Cu") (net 7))
 (segment (start 86.385 72.415) (end 86.385 74.27) (width 0.5) (layer "B.Cu") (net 7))
 (segment (start 86.36 72.39) (end 86.385 72.415) (width 0.5) (layer "B.Cu") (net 7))
 (segment (start 89.8525 76.2) (end 90.805 76.2) (width 0.5) (layer "B.Cu") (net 10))
 (segment (start 91.465 75.54) (end 91.465 74.27) (width 0.5) (layer "B.Cu") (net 10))
 (segment (start 88.925 77.1275) (end 89.8525 76.2) (width 0.5) (layer "B.Cu") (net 10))
 (segment (start 90.805 76.2) (end 91.465 75.54) (width 0.5) (layer "B.Cu") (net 10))
 (segment (start 88.925 78.715) (end 88.925 77.1275) (width 0.5) (layer "B.Cu") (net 10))
 (segment (start 81.305 74.905) (end 81.305 78.715) (width 0.5) (layer "B.Cu") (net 8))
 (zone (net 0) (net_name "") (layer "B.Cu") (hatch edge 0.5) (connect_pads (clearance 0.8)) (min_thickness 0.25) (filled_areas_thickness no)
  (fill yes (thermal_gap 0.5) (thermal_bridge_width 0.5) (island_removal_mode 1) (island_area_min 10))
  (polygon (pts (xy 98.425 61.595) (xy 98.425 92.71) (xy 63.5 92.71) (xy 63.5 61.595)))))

